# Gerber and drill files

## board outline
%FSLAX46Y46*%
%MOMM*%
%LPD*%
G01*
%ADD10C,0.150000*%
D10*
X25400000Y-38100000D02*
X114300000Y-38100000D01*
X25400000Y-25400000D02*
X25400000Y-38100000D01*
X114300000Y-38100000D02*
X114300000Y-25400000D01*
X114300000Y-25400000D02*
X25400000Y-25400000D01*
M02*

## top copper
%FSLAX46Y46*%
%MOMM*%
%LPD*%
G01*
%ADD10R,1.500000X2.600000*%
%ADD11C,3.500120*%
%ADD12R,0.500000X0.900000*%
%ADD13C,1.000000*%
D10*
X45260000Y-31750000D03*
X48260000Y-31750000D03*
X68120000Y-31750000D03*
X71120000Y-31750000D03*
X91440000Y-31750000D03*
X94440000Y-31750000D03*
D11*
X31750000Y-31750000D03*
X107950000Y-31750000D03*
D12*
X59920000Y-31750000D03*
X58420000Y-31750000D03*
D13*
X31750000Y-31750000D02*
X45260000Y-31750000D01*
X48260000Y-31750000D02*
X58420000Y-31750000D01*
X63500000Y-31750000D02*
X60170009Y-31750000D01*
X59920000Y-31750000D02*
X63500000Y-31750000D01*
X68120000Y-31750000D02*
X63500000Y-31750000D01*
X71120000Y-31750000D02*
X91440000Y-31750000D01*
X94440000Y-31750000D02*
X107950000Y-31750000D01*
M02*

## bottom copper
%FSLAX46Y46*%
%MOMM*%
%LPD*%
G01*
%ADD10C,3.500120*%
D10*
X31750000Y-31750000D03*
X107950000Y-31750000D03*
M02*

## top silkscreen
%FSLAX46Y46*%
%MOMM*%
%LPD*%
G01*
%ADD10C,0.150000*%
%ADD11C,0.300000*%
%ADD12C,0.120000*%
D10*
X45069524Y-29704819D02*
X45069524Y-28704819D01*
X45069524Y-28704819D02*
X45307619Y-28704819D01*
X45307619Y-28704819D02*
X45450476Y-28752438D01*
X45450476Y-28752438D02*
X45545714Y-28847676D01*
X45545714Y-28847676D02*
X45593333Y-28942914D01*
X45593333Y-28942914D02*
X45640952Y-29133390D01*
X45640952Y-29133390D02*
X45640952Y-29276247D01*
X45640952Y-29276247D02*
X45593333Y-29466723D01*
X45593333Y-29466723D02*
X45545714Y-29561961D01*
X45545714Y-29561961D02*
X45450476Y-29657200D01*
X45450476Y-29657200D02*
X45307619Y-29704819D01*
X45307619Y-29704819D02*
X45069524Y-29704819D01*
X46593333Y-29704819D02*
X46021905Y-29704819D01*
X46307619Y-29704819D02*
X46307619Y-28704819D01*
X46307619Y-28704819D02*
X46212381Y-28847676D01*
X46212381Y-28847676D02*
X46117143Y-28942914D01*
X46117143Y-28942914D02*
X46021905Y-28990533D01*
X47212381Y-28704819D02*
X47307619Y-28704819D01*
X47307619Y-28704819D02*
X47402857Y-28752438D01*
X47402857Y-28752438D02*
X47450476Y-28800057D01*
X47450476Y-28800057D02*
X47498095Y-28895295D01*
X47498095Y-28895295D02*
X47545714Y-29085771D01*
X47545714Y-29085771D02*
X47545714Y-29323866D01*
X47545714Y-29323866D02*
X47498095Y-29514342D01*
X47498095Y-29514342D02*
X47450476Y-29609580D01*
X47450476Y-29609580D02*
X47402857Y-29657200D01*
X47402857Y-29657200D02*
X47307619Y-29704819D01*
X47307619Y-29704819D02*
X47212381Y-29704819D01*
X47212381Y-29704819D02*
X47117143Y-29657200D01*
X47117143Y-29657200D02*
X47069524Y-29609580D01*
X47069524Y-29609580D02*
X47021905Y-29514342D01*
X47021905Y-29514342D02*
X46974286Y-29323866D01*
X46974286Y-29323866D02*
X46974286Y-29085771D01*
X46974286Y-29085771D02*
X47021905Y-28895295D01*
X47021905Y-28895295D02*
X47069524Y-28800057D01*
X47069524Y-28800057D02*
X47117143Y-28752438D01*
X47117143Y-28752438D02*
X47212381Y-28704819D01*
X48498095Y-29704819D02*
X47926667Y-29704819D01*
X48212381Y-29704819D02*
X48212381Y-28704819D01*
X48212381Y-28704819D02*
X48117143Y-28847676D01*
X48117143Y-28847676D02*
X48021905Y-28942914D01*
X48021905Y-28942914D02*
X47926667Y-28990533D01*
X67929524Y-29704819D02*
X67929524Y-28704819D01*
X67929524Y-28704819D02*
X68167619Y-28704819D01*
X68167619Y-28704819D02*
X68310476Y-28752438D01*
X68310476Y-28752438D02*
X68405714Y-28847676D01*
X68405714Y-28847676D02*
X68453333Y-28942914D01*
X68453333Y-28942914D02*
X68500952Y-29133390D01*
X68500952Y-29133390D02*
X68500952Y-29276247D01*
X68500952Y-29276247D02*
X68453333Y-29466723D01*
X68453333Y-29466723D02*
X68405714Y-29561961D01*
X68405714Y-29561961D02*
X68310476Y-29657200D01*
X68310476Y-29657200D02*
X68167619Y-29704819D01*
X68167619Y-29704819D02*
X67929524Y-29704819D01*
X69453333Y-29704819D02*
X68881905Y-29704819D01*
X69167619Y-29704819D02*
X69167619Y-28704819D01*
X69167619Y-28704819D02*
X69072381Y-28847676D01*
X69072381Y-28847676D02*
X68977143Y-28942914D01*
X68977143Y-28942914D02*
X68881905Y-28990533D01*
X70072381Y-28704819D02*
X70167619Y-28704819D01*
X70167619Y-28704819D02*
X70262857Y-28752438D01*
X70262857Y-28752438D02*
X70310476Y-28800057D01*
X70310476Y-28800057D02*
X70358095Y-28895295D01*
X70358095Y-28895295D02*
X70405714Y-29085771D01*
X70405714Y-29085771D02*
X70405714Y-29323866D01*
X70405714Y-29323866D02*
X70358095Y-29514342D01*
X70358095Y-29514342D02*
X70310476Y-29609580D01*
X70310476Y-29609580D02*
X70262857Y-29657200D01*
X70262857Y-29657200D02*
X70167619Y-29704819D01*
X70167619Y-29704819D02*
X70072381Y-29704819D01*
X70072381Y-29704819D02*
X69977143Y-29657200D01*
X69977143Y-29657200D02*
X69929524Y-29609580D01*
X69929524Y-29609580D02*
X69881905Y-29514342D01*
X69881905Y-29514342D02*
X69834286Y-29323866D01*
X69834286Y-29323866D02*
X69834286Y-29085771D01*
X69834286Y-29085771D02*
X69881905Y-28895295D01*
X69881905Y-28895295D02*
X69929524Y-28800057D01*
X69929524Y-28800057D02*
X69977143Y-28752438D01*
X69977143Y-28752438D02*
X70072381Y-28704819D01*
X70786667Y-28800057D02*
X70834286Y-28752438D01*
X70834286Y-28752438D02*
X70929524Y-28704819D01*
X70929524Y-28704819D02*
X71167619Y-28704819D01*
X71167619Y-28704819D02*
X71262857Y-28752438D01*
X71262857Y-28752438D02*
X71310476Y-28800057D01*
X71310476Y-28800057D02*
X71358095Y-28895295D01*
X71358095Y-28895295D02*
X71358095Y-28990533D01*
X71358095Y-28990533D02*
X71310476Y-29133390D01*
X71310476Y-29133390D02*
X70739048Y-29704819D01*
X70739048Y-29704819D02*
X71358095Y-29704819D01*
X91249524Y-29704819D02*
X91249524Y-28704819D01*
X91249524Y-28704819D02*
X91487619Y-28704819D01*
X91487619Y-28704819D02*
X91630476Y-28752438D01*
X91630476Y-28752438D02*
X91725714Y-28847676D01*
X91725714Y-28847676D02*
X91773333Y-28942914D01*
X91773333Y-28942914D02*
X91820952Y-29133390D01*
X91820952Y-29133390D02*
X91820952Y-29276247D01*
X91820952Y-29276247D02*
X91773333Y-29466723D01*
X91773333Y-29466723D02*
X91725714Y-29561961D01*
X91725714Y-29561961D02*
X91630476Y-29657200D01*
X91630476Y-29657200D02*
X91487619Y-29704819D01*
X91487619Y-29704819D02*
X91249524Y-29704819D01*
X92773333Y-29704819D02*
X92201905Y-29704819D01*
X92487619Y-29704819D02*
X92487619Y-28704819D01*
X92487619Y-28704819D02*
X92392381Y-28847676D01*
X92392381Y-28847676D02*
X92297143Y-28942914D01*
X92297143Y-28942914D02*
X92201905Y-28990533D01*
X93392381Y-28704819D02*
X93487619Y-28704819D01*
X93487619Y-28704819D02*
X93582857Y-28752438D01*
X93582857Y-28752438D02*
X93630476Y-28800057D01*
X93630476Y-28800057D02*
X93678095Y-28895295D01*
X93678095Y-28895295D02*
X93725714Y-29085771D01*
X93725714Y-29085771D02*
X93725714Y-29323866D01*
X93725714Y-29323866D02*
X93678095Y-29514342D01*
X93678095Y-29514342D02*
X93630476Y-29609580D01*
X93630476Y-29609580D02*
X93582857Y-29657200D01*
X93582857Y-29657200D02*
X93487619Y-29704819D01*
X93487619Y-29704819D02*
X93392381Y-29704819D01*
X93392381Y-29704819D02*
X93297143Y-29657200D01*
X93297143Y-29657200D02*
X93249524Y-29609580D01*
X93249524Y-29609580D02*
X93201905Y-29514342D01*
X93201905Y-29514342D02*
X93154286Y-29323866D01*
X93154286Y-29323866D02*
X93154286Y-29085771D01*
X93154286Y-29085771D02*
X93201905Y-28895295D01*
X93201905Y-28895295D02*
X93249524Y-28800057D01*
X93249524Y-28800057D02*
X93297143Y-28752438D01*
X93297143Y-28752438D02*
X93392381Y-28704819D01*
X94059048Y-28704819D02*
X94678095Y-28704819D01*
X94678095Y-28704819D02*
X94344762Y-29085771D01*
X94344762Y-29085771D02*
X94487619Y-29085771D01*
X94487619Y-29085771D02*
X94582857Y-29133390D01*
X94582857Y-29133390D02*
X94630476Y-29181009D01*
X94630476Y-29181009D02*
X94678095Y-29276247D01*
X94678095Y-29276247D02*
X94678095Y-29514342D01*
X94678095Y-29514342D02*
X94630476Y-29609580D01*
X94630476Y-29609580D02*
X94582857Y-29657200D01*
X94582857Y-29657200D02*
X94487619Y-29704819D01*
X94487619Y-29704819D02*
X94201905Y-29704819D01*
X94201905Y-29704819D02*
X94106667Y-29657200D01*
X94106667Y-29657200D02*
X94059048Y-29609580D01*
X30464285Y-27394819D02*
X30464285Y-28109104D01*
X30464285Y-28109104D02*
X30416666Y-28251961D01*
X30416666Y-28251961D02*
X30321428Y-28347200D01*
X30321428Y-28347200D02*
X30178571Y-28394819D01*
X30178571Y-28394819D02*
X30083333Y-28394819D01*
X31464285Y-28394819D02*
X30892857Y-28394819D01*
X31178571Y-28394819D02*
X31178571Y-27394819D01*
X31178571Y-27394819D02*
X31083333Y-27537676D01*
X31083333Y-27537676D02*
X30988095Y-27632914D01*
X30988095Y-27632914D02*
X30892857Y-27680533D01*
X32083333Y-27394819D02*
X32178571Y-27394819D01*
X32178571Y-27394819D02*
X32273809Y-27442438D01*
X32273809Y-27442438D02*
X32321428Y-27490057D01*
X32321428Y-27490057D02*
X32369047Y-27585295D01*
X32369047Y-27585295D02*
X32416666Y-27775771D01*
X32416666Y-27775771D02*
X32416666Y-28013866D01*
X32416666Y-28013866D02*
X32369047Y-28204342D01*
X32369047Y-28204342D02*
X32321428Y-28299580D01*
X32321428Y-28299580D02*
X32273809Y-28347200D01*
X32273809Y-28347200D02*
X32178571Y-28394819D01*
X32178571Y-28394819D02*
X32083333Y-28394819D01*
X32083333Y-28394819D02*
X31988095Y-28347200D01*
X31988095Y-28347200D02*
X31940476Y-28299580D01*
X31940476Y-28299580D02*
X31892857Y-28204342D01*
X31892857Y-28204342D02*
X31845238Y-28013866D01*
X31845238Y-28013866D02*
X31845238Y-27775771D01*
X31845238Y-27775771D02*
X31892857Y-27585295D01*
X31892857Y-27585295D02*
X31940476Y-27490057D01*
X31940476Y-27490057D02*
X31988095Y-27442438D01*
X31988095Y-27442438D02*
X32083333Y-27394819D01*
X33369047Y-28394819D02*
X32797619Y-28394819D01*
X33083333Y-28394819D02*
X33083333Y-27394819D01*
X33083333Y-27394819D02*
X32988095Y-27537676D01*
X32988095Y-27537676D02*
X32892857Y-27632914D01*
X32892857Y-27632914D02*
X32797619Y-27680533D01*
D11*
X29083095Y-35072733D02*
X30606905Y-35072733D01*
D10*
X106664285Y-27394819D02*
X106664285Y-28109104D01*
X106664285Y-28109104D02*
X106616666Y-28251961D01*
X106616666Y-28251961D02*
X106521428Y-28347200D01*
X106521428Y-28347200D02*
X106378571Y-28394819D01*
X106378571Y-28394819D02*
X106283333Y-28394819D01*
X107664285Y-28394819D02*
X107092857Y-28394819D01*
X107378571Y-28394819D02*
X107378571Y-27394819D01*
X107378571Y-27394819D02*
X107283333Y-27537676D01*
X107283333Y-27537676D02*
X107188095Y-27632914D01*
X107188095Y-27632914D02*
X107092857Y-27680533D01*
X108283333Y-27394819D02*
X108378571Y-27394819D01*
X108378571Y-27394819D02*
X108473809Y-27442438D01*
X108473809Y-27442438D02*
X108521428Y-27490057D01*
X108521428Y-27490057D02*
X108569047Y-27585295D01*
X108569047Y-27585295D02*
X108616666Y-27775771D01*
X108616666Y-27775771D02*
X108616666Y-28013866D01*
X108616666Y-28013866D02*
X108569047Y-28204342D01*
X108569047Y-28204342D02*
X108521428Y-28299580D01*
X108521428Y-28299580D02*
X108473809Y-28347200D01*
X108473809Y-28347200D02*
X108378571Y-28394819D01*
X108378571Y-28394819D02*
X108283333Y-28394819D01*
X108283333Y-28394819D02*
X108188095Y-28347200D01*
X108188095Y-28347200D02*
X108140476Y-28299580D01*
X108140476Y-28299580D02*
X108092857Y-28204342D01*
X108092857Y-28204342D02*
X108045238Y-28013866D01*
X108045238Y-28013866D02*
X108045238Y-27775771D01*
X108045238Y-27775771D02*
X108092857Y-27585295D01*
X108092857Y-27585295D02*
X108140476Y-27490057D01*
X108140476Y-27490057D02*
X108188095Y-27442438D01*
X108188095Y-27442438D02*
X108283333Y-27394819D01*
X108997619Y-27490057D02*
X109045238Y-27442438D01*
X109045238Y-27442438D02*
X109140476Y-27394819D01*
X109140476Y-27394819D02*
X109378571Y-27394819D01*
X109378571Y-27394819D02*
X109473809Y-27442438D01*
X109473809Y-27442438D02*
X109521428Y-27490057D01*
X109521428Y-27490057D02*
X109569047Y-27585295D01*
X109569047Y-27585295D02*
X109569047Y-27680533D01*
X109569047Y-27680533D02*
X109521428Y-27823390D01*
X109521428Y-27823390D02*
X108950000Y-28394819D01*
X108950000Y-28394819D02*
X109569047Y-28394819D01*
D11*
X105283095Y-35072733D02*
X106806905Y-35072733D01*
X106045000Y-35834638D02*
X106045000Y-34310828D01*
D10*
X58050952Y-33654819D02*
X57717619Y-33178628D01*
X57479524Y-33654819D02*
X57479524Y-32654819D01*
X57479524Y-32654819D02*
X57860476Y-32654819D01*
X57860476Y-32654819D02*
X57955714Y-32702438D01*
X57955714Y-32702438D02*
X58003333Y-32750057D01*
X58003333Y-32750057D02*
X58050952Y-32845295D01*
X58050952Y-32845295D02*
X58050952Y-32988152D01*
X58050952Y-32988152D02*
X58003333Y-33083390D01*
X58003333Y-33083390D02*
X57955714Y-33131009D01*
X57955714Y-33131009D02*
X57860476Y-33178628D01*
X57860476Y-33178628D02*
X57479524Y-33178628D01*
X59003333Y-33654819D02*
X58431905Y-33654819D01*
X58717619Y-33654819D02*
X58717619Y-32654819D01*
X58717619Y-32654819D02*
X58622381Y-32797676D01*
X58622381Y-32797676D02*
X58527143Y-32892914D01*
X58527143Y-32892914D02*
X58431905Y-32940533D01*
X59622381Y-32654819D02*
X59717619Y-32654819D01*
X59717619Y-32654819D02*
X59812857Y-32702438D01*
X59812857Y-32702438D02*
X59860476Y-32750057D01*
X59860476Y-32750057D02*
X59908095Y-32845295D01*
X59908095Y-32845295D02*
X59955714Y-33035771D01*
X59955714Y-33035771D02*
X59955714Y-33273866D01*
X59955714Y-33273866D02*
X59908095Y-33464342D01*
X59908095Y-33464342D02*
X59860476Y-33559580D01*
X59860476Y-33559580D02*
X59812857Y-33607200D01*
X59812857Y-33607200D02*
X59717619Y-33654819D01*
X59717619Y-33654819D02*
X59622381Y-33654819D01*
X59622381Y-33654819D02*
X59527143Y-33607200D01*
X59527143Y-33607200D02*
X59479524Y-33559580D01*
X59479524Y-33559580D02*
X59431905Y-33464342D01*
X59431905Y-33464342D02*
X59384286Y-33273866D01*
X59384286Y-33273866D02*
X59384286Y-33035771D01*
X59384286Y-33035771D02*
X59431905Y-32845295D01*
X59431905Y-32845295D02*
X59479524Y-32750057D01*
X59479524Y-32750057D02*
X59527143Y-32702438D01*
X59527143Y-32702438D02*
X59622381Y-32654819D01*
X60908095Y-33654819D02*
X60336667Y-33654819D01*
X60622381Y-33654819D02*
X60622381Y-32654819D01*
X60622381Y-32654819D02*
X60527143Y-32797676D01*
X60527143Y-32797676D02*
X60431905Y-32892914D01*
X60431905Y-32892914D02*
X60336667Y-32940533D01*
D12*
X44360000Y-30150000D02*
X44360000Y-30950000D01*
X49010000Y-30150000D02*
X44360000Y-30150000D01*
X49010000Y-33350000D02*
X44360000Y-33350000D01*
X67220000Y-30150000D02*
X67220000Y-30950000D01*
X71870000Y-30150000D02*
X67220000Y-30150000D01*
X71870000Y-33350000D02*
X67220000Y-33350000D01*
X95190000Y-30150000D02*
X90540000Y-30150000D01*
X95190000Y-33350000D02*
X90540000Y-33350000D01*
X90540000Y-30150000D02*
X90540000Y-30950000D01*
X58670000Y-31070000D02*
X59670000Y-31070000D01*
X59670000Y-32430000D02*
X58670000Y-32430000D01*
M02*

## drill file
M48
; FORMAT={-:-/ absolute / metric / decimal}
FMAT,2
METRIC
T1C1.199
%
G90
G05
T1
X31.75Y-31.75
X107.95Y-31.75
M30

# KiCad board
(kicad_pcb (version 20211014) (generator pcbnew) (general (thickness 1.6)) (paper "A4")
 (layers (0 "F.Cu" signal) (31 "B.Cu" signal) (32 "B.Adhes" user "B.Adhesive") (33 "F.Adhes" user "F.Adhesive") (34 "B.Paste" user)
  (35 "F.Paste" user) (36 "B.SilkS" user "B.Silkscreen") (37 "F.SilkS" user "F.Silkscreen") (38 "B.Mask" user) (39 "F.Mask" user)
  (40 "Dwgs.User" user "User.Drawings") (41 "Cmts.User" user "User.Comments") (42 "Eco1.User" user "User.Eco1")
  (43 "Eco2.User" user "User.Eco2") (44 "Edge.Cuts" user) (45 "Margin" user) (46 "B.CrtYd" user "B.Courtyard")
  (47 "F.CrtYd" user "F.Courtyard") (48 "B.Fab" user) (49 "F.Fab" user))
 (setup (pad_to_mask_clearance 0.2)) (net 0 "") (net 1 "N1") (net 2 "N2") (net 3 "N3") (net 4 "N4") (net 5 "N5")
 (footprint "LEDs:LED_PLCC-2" (layer "F.Cu") (at 46.76 31.75)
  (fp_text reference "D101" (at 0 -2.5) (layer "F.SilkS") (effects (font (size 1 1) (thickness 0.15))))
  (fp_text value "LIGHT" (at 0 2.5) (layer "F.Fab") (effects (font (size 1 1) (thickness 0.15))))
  (fp_line (start -2.4 -1.6) (end -2.4 -0.8) (layer "F.SilkS") (width 0.12))
  (fp_line (start 2.25 -1.6) (end -2.4 -1.6) (layer "F.SilkS") (width 0.12))
  (fp_line (start 2.25 1.6) (end -2.4 1.6) (layer "F.SilkS") (width 0.12))
  (pad "1" smd rect locked (at -1.5 0) (size 1.5 2.6) (layers "F.Cu" "F.Paste" "F.Mask") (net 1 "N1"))
  (pad "2" smd rect locked (at 1.5 0) (size 1.5 2.6) (layers "F.Cu" "F.Paste" "F.Mask") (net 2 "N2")))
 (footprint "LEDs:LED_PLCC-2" (layer "F.Cu") (at 69.62 31.75)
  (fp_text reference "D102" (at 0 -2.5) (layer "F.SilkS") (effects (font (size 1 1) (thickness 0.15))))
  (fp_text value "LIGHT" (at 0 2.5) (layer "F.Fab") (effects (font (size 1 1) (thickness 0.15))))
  (fp_line (start -2.4 -1.6) (end -2.4 -0.8) (layer "F.SilkS") (width 0.12))
  (fp_line (start 2.25 -1.6) (end -2.4 -1.6) (layer "F.SilkS") (width 0.12))
  (fp_line (start 2.25 1.6) (end -2.4 1.6) (layer "F.SilkS") (width 0.12))
  (pad "1" smd rect locked (at -1.5 0) (size 1.5 2.6) (layers "F.Cu" "F.Paste" "F.Mask") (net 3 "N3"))
  (pad "2" smd rect locked (at 1.5 0) (size 1.5 2.6) (layers "F.Cu" "F.Paste" "F.Mask") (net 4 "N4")))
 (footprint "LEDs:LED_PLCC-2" (layer "F.Cu") (at 92.94 31.75)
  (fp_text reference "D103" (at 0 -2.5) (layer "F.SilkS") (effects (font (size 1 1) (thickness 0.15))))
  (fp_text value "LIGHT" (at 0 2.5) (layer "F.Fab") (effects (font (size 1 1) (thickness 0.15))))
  (fp_line (start 2.25 -1.6) (end -2.4 -1.6) (layer "F.SilkS") (width 0.12))
  (fp_line (start 2.25 1.6) (end -2.4 1.6) (layer "F.SilkS") (width 0.12))
  (fp_line (start -2.4 -1.6) (end -2.4 -0.8) (layer "F.SilkS") (width 0.12))
  (pad "1" smd rect locked (at -1.5 0) (size 1.5 2.6) (layers "F.Cu" "F.Paste" "F.Mask") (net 4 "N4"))
  (pad "2" smd rect locked (at 1.5 0) (size 1.5 2.6) (layers "F.Cu" "F.Paste" "F.Mask") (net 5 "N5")))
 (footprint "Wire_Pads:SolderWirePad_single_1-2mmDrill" (layer "F.Cu") (at 31.75 31.75)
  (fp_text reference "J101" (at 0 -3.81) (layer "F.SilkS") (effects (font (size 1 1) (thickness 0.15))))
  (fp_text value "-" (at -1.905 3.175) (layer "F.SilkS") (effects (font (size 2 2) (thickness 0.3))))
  (pad "1" thru_hole circle locked (at 0 0) (size 3.50012 3.50012) (drill 1.19888) (layers *.Cu *.Mask) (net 1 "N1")))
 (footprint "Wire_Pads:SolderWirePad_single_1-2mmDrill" (layer "F.Cu") (at 107.95 31.75)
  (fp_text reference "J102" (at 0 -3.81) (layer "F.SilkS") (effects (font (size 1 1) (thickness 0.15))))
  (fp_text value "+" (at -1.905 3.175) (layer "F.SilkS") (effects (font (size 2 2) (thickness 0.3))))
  (pad "1" thru_hole circle locked (at 0 0) (size 3.50012 3.50012) (drill 1.19888) (layers *.Cu *.Mask) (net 5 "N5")))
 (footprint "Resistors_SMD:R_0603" (layer "F.Cu") (at 59.17 31.75 180)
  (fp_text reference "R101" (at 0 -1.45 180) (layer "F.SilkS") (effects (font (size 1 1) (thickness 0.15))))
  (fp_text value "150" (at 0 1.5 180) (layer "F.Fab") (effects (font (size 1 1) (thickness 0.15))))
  (fp_line (start 0.5 0.68) (end -0.5 0.68) (layer "F.SilkS") (width 0.12))
  (fp_line (start -0.5 -0.68) (end 0.5 -0.68) (layer "F.SilkS") (width 0.12))
  (pad "1" smd rect locked (at -0.75 0 180) (size 0.5 0.9) (layers "F.Cu" "F.Paste" "F.Mask") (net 3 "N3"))
  (pad "2" smd rect locked (at 0.75 0 180) (size 0.5 0.9) (layers "F.Cu" "F.Paste" "F.Mask") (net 2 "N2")))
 (gr_line (start 25.4 38.1) (end 114.3 38.1) (layer "Edge.Cuts") (width 0.15))
 (gr_line (start 25.4 25.4) (end 25.4 38.1) (layer "Edge.Cuts") (width 0.15))
 (gr_line (start 114.3 38.1) (end 114.3 25.4) (layer "Edge.Cuts") (width 0.15))
 (gr_line (start 114.3 25.4) (end 25.4 25.4) (layer "Edge.Cuts") (width 0.15))
 (segment (start 31.75 31.75) (end 45.26 31.75) (width 1) (layer "F.Cu") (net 1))
 (segment (start 48.26 31.75) (end 58.42 31.75) (width 1) (layer "F.Cu") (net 2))
 (segment (start 63.5 31.75) (end 60.170009 31.75) (width 1) (layer "F.Cu") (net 3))
 (segment (start 59.92 31.75) (end 63.5 31.75) (width 1) (layer "F.Cu") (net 3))
 (segment (start 68.12 31.75) (end 63.5 31.75) (width 1) (layer "F.Cu") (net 3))
 (segment (start 71.12 31.75) (end 91.44 31.75) (width 1) (layer "F.Cu") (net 4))
 (segment (start 94.44 31.75) (end 107.95 31.75) (width 1) (layer "F.Cu") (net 5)))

